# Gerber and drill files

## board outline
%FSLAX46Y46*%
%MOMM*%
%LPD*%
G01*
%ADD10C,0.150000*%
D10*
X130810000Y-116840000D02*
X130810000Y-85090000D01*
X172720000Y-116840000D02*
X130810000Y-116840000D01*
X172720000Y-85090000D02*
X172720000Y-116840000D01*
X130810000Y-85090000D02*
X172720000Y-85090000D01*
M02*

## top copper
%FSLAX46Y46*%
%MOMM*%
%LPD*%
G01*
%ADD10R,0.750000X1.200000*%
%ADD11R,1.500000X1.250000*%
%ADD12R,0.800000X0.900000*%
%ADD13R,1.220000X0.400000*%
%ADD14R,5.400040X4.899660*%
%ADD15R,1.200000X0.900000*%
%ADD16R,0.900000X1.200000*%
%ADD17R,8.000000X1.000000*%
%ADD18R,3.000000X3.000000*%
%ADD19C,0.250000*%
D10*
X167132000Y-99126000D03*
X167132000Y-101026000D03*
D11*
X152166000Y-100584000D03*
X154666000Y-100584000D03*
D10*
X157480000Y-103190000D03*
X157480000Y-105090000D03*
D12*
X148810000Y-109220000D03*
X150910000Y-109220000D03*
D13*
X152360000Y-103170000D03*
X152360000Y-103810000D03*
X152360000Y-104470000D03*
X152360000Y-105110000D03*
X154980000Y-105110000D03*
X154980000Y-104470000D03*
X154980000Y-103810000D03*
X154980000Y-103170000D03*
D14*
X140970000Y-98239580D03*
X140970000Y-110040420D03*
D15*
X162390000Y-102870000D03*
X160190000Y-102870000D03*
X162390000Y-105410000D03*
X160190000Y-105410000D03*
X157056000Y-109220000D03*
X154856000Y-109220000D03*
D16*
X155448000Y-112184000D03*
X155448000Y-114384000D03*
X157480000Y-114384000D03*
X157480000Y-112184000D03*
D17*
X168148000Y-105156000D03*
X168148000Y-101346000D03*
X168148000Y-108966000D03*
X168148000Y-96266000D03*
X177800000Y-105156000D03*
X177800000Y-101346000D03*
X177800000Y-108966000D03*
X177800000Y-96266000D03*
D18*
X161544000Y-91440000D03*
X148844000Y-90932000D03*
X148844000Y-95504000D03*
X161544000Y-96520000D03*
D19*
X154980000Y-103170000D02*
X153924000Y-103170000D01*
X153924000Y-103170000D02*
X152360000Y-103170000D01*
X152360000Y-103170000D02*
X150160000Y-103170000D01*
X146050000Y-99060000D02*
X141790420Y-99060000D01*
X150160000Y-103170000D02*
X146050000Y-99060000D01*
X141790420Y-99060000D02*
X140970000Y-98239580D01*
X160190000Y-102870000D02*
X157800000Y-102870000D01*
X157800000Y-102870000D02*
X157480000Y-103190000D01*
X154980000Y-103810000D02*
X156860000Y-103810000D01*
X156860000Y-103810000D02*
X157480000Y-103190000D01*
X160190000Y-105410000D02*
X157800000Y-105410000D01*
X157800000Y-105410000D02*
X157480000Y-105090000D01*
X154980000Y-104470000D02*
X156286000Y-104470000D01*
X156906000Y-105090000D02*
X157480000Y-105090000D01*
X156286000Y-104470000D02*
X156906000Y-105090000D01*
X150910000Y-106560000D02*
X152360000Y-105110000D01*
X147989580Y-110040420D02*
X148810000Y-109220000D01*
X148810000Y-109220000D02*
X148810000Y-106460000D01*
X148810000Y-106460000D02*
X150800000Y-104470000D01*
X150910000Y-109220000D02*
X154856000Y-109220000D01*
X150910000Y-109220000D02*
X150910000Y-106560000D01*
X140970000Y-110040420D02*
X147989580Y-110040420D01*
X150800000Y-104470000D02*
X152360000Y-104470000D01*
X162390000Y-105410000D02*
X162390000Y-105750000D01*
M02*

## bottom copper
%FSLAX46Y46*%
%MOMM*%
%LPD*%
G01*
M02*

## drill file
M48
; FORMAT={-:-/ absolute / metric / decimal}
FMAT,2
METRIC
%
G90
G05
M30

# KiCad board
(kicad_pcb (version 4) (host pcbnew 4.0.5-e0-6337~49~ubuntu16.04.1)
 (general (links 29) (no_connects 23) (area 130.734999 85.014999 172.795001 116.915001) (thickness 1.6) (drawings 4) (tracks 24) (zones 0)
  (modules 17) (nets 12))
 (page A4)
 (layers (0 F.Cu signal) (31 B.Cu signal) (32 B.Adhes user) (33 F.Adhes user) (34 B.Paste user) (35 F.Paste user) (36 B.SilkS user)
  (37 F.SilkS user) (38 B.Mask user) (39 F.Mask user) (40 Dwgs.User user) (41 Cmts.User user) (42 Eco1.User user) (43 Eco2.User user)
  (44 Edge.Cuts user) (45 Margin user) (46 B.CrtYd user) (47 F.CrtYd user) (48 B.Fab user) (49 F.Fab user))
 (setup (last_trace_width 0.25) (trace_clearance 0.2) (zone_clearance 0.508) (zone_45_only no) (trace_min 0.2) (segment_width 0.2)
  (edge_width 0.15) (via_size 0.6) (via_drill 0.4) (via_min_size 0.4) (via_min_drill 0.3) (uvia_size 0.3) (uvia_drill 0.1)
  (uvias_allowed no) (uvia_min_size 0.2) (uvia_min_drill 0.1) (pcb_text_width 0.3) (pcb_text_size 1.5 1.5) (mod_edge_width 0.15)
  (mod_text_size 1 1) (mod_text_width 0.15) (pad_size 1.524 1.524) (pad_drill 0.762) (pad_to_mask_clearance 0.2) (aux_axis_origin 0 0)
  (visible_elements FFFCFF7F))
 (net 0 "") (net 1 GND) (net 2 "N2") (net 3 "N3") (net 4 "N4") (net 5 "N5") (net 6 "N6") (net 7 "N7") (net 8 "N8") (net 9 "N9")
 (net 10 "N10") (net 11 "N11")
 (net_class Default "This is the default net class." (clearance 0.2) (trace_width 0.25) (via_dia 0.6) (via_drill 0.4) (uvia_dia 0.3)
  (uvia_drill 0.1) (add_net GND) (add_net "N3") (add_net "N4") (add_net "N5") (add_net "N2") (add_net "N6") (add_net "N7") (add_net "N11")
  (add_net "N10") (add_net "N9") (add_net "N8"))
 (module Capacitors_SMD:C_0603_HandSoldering (layer F.Cu) (at 167.132 100.076 270)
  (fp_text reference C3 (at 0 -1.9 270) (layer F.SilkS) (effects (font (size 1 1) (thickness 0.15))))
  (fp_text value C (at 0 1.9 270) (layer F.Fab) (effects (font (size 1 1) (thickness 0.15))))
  (pad 1 smd rect (at -0.95 0 270) (size 1.2 0.75) (layers F.Cu F.Paste F.Mask) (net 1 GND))
  (pad 2 smd rect (at 0.95 0 270) (size 1.2 0.75) (layers F.Cu F.Paste F.Mask) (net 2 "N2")))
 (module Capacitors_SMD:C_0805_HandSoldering (layer F.Cu) (at 153.416 100.584)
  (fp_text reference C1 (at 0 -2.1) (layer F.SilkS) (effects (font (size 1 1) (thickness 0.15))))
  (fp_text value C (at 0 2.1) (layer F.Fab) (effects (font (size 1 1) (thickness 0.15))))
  (pad 1 smd rect (at -1.25 0) (size 1.5 1.25) (layers F.Cu F.Paste F.Mask) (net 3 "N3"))
  (pad 2 smd rect (at 1.25 0) (size 1.5 1.25) (layers F.Cu F.Paste F.Mask) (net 1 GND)))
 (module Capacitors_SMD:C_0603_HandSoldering (layer F.Cu) (at 157.48 104.14 270)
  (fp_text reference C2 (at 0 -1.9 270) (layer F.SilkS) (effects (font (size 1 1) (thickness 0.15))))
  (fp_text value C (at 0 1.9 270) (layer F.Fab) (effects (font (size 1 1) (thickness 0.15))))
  (pad 1 smd rect (at -0.95 0 270) (size 1.2 0.75) (layers F.Cu F.Paste F.Mask) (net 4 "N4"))
  (pad 2 smd rect (at 0.95 0 270) (size 1.2 0.75) (layers F.Cu F.Paste F.Mask) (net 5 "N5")))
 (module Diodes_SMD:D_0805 (layer F.Cu) (at 149.86 109.22)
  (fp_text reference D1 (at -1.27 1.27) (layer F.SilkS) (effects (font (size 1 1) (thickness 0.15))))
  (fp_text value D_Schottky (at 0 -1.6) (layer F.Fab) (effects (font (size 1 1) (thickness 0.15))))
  (pad 1 smd rect (at -1.05 0) (size 0.8 0.9) (layers F.Cu F.Paste F.Mask) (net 2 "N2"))
  (pad 2 smd rect (at 1.05 0) (size 0.8 0.9) (layers F.Cu F.Paste F.Mask) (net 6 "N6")))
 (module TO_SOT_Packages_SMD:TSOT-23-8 (layer F.Cu) (at 153.67 104.14)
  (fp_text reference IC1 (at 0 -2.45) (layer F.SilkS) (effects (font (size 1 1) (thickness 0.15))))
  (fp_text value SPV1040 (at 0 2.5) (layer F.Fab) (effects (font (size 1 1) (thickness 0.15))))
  (pad 1 smd rect (at -1.31 -0.97) (size 1.22 0.4) (layers F.Cu F.Paste F.Mask) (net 3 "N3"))
  (pad 2 smd rect (at -1.31 -0.33) (size 1.22 0.4) (layers F.Cu F.Paste F.Mask) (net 1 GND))
  (pad 3 smd rect (at -1.31 0.33) (size 1.22 0.4) (layers F.Cu F.Paste F.Mask) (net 6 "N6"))
  (pad 4 smd rect (at -1.31 0.97) (size 1.22 0.4) (layers F.Cu F.Paste F.Mask) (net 2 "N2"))
  (pad 5 smd rect (at 1.31 0.97) (size 1.22 0.4) (layers F.Cu F.Paste F.Mask) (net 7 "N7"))
  (pad 6 smd rect (at 1.31 0.33) (size 1.22 0.4) (layers F.Cu F.Paste F.Mask) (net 5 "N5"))
  (pad 7 smd rect (at 1.31 -0.33) (size 1.22 0.4) (layers F.Cu F.Paste F.Mask) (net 4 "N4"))
  (pad 8 smd rect (at 1.31 -0.97) (size 1.22 0.4) (layers F.Cu F.Paste F.Mask) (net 3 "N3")))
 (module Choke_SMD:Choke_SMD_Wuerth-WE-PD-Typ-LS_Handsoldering (layer F.Cu) (at 140.97 104.14 270)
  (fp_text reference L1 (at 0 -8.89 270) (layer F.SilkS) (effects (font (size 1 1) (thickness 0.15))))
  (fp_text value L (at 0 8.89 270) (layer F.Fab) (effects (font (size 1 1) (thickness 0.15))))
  (pad 1 smd rect (at -5.90042 0 270) (size 4.89966 5.40004) (layers F.Cu F.Paste F.Mask) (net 3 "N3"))
  (pad 2 smd rect (at 5.90042 0 270) (size 4.89966 5.40004) (layers F.Cu F.Paste F.Mask) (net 6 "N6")))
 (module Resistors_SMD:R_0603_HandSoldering (layer F.Cu) (at 161.29 102.87 180)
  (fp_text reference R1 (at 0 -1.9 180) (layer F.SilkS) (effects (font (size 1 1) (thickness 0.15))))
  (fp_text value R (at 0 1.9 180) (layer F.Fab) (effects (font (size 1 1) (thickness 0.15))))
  (pad 1 smd rect (at -1.1 0 180) (size 1.2 0.9) (layers F.Cu F.Paste F.Mask) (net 2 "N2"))
  (pad 2 smd rect (at 1.1 0 180) (size 1.2 0.9) (layers F.Cu F.Paste F.Mask) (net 4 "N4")))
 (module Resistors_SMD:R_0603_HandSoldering (layer F.Cu) (at 161.29 105.41 180)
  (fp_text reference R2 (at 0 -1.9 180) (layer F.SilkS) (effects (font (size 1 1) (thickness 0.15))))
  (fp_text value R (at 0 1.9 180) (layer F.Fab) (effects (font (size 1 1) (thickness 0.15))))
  (pad 1 smd rect (at -1.1 0 180) (size 1.2 0.9) (layers F.Cu F.Paste F.Mask) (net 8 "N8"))
  (pad 2 smd rect (at 1.1 0 180) (size 1.2 0.9) (layers F.Cu F.Paste F.Mask) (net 5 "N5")))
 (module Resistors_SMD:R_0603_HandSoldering (layer F.Cu) (at 155.956 109.22 180)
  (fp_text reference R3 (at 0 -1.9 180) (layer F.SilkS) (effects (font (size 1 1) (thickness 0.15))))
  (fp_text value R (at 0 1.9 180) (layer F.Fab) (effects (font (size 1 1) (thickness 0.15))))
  (pad 1 smd rect (at -1.1 0 180) (size 1.2 0.9) (layers F.Cu F.Paste F.Mask) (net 8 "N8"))
  (pad 2 smd rect (at 1.1 0 180) (size 1.2 0.9) (layers F.Cu F.Paste F.Mask) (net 2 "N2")))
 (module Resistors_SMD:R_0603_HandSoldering (layer F.Cu) (at 155.448 113.284 270)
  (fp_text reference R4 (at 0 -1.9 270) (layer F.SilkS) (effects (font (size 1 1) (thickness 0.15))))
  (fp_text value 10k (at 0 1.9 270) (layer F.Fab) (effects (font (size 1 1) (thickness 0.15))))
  (pad 1 smd rect (at -1.1 0 270) (size 1.2 0.9) (layers F.Cu F.Paste F.Mask) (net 8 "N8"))
  (pad 2 smd rect (at 1.1 0 270) (size 1.2 0.9) (layers F.Cu F.Paste F.Mask) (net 7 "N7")))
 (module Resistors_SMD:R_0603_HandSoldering (layer F.Cu) (at 157.48 113.284 90)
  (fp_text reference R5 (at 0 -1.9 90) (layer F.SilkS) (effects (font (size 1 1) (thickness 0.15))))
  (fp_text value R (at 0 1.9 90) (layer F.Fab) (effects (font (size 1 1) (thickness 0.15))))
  (pad 1 smd rect (at -1.1 0 90) (size 1.2 0.9) (layers F.Cu F.Paste F.Mask) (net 7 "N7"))
  (pad 2 smd rect (at 1.1 0 90) (size 1.2 0.9) (layers F.Cu F.Paste F.Mask) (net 1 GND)))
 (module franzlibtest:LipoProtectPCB (layer F.Cu) (at 168.148 110.236)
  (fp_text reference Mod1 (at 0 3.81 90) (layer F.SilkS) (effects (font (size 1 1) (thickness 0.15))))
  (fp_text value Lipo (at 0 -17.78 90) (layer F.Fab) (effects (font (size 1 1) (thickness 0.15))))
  (pad 3 smd rect (at 0 -5.08) (size 8 1) (layers F.Cu F.Paste F.Mask) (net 1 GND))
  (pad 4 smd rect (at 0 -8.89) (size 8 1) (layers F.Cu F.Paste F.Mask) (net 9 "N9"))
  (pad 2 smd rect (at 0 -1.27) (size 8 1) (layers F.Cu F.Paste F.Mask) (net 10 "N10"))
  (pad 1 smd rect (at 0 -13.97) (size 8 1) (layers F.Cu F.Paste F.Mask) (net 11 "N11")))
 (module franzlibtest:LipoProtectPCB (layer F.Cu) (at 177.8 110.236)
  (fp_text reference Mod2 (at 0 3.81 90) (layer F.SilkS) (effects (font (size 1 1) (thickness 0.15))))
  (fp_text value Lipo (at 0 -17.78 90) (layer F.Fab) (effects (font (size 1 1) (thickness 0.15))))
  (pad 3 smd rect (at 0 -5.08) (size 8 1) (layers F.Cu F.Paste F.Mask) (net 1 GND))
  (pad 4 smd rect (at 0 -8.89) (size 8 1) (layers F.Cu F.Paste F.Mask) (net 8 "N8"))
  (pad 2 smd rect (at 0 -1.27) (size 8 1) (layers F.Cu F.Paste F.Mask) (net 10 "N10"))
  (pad 1 smd rect (at 0 -13.97) (size 8 1) (layers F.Cu F.Paste F.Mask) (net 11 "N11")))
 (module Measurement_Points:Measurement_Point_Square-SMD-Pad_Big (layer F.Cu) (at 161.544 91.44)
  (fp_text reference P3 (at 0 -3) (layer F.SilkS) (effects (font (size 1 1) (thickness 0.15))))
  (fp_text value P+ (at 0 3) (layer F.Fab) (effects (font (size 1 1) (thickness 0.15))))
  (pad 1 smd rect (at 0 0) (size 3 3) (layers F.Cu F.Mask) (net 9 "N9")))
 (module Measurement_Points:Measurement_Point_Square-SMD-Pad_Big (layer F.Cu) (at 148.844 90.932)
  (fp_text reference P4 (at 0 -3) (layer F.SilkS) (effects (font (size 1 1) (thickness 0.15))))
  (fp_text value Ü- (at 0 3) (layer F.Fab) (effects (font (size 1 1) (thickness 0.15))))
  (pad 1 smd rect (at 0 0) (size 3 3) (layers F.Cu F.Mask) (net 1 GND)))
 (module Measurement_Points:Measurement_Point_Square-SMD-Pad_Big (layer F.Cu) (at 148.844 95.504)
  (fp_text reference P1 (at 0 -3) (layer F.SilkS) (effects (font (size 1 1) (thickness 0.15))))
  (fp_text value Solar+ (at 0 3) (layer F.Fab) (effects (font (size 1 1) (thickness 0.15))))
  (pad 1 smd rect (at 0 0) (size 3 3) (layers F.Cu F.Mask) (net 3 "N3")))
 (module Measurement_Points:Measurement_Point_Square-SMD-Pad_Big (layer F.Cu) (at 161.544 96.52)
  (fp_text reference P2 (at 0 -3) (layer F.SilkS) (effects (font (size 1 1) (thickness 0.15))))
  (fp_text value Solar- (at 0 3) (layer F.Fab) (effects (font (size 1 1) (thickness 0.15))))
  (pad 1 smd rect (at 0 0) (size 3 3) (layers F.Cu F.Mask) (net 1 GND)))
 (gr_line (start 130.81 116.84) (end 130.81 85.09) (angle 90) (layer Edge.Cuts) (width 0.15))
 (gr_line (start 172.72 116.84) (end 130.81 116.84) (angle 90) (layer Edge.Cuts) (width 0.15))
 (gr_line (start 172.72 85.09) (end 172.72 116.84) (angle 90) (layer Edge.Cuts) (width 0.15))
 (gr_line (start 130.81 85.09) (end 172.72 85.09) (angle 90) (layer Edge.Cuts) (width 0.15))
 (segment (start 154.98 103.17) (end 153.924 103.17) (width 0.25) (layer F.Cu) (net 3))
 (segment (start 153.924 103.17) (end 152.36 103.17) (width 0.25) (layer F.Cu) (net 3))
 (segment (start 152.36 103.17) (end 150.16 103.17) (width 0.25) (layer F.Cu) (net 3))
 (segment (start 146.05 99.06) (end 141.79042 99.06) (width 0.25) (layer F.Cu) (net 3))
 (segment (start 150.16 103.17) (end 146.05 99.06) (width 0.25) (layer F.Cu) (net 3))
 (segment (start 141.79042 99.06) (end 140.97 98.23958) (width 0.25) (layer F.Cu) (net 3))
 (segment (start 160.19 102.87) (end 157.8 102.87) (width 0.25) (layer F.Cu) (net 4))
 (segment (start 157.8 102.87) (end 157.48 103.19) (width 0.25) (layer F.Cu) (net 4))
 (segment (start 154.98 103.81) (end 156.86 103.81) (width 0.25) (layer F.Cu) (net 4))
 (segment (start 156.86 103.81) (end 157.48 103.19) (width 0.25) (layer F.Cu) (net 4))
 (segment (start 160.19 105.41) (end 157.8 105.41) (width 0.25) (layer F.Cu) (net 5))
 (segment (start 157.8 105.41) (end 157.48 105.09) (width 0.25) (layer F.Cu) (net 5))
 (segment (start 154.98 104.47) (end 156.286 104.47) (width 0.25) (layer F.Cu) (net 5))
 (segment (start 156.906 105.09) (end 157.48 105.09) (width 0.25) (layer F.Cu) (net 5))
 (segment (start 156.286 104.47) (end 156.906 105.09) (width 0.25) (layer F.Cu) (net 5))
 (segment (start 150.91 106.56) (end 152.36 105.11) (width 0.25) (layer F.Cu) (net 2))
 (segment (start 147.98958 110.04042) (end 148.81 109.22) (width 0.25) (layer F.Cu) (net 2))
 (segment (start 148.81 109.22) (end 148.81 106.46) (width 0.25) (layer F.Cu) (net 2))
 (segment (start 148.81 106.46) (end 150.8 104.47) (width 0.25) (layer F.Cu) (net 2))
 (segment (start 150.91 109.22) (end 154.856 109.22) (width 0.25) (layer F.Cu) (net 6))
 (segment (start 150.91 109.22) (end 150.91 106.56) (width 0.25) (layer F.Cu) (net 6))
 (segment (start 140.97 110.04042) (end 147.98958 110.04042) (width 0.25) (layer F.Cu) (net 6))
 (segment (start 150.8 104.47) (end 152.36 104.47) (width 0.25) (layer F.Cu) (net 6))
 (segment (start 162.39 105.41) (end 162.39 105.75) (width 0.25) (layer F.Cu) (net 8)))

